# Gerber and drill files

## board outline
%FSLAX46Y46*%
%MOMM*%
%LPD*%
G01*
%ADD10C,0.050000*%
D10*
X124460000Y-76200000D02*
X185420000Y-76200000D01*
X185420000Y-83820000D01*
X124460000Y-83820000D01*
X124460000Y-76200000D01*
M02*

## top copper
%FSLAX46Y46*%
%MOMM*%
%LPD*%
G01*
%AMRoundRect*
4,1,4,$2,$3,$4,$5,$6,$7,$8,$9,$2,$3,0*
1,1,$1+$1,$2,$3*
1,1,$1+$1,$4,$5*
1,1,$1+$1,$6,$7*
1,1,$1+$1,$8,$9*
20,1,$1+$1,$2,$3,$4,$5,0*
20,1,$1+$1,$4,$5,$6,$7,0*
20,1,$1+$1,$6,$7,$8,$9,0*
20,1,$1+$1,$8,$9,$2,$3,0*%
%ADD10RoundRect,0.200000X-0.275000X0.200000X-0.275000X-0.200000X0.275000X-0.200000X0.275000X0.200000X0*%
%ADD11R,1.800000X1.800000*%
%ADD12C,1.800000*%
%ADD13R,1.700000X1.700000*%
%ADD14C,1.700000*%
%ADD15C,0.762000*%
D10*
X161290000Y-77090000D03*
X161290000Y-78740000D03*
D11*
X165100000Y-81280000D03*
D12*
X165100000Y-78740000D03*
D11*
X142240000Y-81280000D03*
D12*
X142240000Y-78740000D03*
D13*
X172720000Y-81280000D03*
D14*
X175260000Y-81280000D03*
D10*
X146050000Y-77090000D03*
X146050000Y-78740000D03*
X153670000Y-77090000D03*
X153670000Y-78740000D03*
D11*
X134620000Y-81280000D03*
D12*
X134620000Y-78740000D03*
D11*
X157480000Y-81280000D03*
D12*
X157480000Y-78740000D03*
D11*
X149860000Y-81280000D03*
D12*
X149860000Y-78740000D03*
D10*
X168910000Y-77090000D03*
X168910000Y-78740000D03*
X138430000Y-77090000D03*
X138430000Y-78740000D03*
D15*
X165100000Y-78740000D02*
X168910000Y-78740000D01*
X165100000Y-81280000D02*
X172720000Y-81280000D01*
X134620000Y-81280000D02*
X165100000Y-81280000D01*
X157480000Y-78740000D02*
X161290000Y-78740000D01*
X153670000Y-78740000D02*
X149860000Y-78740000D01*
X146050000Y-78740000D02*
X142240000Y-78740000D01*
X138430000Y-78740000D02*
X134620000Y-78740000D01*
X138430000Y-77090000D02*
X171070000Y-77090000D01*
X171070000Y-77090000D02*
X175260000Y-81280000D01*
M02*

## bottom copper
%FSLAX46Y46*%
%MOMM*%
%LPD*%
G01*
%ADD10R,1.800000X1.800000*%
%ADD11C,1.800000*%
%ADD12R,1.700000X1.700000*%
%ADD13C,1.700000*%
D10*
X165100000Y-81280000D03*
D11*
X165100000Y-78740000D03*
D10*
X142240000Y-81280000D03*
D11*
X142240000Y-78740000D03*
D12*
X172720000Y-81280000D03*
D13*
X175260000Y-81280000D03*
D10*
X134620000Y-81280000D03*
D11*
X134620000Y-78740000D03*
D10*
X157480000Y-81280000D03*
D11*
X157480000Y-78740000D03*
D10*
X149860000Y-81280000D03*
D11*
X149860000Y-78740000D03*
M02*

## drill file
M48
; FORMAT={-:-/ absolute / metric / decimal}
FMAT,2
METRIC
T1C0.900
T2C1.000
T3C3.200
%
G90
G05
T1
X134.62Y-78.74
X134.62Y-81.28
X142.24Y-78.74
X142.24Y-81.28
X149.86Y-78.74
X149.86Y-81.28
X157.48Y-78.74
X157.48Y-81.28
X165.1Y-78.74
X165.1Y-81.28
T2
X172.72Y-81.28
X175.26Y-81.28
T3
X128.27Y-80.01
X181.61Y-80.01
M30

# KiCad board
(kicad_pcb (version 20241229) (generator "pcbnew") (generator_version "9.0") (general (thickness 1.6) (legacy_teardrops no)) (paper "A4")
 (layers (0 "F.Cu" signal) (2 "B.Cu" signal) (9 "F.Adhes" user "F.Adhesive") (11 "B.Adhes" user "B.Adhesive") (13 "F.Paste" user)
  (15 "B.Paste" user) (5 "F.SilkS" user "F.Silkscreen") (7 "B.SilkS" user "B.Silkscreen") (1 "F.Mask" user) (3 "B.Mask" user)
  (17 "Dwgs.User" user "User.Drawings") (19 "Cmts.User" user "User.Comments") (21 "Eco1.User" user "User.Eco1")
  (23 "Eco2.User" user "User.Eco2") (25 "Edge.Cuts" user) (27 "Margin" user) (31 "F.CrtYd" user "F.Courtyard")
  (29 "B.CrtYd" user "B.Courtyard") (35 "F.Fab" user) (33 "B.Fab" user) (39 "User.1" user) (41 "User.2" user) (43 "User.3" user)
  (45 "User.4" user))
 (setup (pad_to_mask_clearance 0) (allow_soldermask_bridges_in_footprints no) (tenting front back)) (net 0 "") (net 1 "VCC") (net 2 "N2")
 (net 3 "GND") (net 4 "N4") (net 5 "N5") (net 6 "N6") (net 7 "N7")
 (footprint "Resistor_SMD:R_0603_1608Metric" (layer "F.Cu") (at 161.29 77.915 -90)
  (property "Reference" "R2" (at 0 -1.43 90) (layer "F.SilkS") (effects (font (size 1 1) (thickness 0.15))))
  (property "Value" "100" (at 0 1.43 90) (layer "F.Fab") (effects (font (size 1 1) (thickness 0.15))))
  (pad "1" smd roundrect (at -0.825 0 270) (size 0.8 0.95) (layers "F.Cu" "F.Mask" "F.Paste") (roundrect_rratio 0.25) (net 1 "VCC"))
  (pad "2" smd roundrect (at 0.825 0 270) (size 0.8 0.95) (layers "F.Cu" "F.Mask" "F.Paste") (roundrect_rratio 0.25) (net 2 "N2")))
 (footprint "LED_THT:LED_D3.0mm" (layer "F.Cu") (at 165.1 81.28 90)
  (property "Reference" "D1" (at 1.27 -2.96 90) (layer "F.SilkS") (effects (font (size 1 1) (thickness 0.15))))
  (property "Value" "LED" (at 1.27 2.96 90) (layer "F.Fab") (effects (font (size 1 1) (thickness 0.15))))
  (pad "1" thru_hole rect (at 0 0 90) (size 1.8 1.8) (drill 0.9) (layers "*.Cu" "*.Mask") (remove_unused_layers no) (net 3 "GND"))
  (pad "2" thru_hole circle (at 2.54 0 90) (size 1.8 1.8) (drill 0.9) (layers "*.Cu" "*.Mask") (remove_unused_layers no) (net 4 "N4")))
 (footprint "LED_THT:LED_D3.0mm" (layer "F.Cu") (at 142.24 81.28 90)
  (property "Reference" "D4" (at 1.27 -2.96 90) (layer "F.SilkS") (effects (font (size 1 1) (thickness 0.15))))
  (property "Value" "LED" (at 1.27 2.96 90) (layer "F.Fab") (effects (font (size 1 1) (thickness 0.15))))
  (pad "1" thru_hole rect (at 0 0 90) (size 1.8 1.8) (drill 0.9) (layers "*.Cu" "*.Mask") (remove_unused_layers no) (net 3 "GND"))
  (pad "2" thru_hole circle (at 2.54 0 90) (size 1.8 1.8) (drill 0.9) (layers "*.Cu" "*.Mask") (remove_unused_layers no) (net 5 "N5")))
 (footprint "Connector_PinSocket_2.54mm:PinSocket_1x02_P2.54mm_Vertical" (layer "F.Cu") (at 172.72 81.28 90)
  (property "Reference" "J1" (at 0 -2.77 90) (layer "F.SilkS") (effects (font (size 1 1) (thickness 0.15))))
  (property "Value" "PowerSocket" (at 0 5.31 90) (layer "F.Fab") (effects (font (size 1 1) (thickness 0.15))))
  (pad "1" thru_hole rect (at 0 0 90) (size 1.7 1.7) (drill 1) (layers "*.Cu" "*.Mask") (remove_unused_layers no) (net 3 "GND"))
  (pad "2" thru_hole circle (at 0 2.54 90) (size 1.7 1.7) (drill 1) (layers "*.Cu" "*.Mask") (remove_unused_layers no) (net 1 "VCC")))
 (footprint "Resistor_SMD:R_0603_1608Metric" (layer "F.Cu") (at 146.05 77.915 -90)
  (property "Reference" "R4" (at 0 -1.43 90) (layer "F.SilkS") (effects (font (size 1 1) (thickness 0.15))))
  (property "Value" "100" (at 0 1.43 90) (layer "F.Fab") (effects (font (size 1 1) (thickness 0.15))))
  (pad "1" smd roundrect (at -0.825 0 270) (size 0.8 0.95) (layers "F.Cu" "F.Mask" "F.Paste") (roundrect_rratio 0.25) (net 1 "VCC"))
  (pad "2" smd roundrect (at 0.825 0 270) (size 0.8 0.95) (layers "F.Cu" "F.Mask" "F.Paste") (roundrect_rratio 0.25) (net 5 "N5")))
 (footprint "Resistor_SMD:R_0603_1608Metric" (layer "F.Cu") (at 153.67 77.915 -90)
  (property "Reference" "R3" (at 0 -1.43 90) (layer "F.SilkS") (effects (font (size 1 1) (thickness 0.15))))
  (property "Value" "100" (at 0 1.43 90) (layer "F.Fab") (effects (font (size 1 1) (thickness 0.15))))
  (pad "1" smd roundrect (at -0.825 0 270) (size 0.8 0.95) (layers "F.Cu" "F.Mask" "F.Paste") (roundrect_rratio 0.25) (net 1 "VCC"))
  (pad "2" smd roundrect (at 0.825 0 270) (size 0.8 0.95) (layers "F.Cu" "F.Mask" "F.Paste") (roundrect_rratio 0.25) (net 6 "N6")))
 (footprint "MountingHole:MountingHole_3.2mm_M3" (layer "F.Cu") (at 128.27 80.01)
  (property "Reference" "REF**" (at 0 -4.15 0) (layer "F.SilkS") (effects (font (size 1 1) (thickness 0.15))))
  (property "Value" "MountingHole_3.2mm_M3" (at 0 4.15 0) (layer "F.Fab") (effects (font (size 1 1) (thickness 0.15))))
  (pad "" np_thru_hole circle (at 0 0) (size 3.2 3.2) (drill 3.2) (layers "*.Cu" "*.Mask")))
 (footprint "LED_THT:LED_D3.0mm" (layer "F.Cu") (at 134.62 81.28 90)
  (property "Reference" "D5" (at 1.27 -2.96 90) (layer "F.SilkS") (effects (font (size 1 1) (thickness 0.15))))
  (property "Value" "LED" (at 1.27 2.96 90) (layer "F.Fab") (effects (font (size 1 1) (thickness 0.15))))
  (pad "1" thru_hole rect (at 0 0 90) (size 1.8 1.8) (drill 0.9) (layers "*.Cu" "*.Mask") (remove_unused_layers no) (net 3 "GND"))
  (pad "2" thru_hole circle (at 2.54 0 90) (size 1.8 1.8) (drill 0.9) (layers "*.Cu" "*.Mask") (remove_unused_layers no) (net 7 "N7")))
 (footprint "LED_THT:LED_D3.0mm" (layer "F.Cu") (at 157.48 81.28 90)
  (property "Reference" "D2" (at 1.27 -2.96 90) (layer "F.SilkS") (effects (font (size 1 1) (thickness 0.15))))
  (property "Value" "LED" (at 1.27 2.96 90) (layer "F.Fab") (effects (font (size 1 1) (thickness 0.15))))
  (pad "1" thru_hole rect (at 0 0 90) (size 1.8 1.8) (drill 0.9) (layers "*.Cu" "*.Mask") (remove_unused_layers no) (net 3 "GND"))
  (pad "2" thru_hole circle (at 2.54 0 90) (size 1.8 1.8) (drill 0.9) (layers "*.Cu" "*.Mask") (remove_unused_layers no) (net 2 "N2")))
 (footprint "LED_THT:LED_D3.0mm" (layer "F.Cu") (at 149.86 81.28 90)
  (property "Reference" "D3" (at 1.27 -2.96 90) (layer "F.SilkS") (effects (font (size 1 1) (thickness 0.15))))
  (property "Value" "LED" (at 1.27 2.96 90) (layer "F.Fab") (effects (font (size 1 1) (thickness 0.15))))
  (pad "1" thru_hole rect (at 0 0 90) (size 1.8 1.8) (drill 0.9) (layers "*.Cu" "*.Mask") (remove_unused_layers no) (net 3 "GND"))
  (pad "2" thru_hole circle (at 2.54 0 90) (size 1.8 1.8) (drill 0.9) (layers "*.Cu" "*.Mask") (remove_unused_layers no) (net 6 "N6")))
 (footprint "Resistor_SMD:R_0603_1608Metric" (layer "F.Cu") (at 168.91 77.915 -90)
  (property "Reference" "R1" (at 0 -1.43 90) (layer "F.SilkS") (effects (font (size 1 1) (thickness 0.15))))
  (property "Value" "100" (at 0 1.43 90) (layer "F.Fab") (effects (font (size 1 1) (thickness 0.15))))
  (pad "1" smd roundrect (at -0.825 0 270) (size 0.8 0.95) (layers "F.Cu" "F.Mask" "F.Paste") (roundrect_rratio 0.25) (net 1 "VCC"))
  (pad "2" smd roundrect (at 0.825 0 270) (size 0.8 0.95) (layers "F.Cu" "F.Mask" "F.Paste") (roundrect_rratio 0.25) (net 4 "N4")))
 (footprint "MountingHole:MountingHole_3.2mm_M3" (layer "F.Cu") (at 181.61 80.01)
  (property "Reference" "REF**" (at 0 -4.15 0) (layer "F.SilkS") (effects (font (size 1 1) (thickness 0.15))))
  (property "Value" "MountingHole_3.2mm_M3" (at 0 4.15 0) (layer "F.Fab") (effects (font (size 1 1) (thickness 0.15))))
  (pad "" np_thru_hole circle (at 0 0) (size 3.2 3.2) (drill 3.2) (layers "*.Cu" "*.Mask")))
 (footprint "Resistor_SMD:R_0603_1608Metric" (layer "F.Cu") (at 138.43 77.915 -90)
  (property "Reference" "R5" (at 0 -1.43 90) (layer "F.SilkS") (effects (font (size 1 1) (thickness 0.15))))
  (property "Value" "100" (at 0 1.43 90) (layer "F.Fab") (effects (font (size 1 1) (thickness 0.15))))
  (pad "1" smd roundrect (at -0.825 0 270) (size 0.8 0.95) (layers "F.Cu" "F.Mask" "F.Paste") (roundrect_rratio 0.25) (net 1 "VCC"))
  (pad "2" smd roundrect (at 0.825 0 270) (size 0.8 0.95) (layers "F.Cu" "F.Mask" "F.Paste") (roundrect_rratio 0.25) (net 7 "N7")))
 (gr_rect (start 124.46 76.2) (end 185.42 83.82) (stroke (width 0.05) (type default)) (fill no) (layer "Edge.Cuts"))
 (segment (start 165.1 78.74) (end 168.91 78.74) (width 0.762) (layer "F.Cu") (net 4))
 (segment (start 165.1 81.28) (end 172.72 81.28) (width 0.762) (layer "F.Cu") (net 3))
 (segment (start 134.62 81.28) (end 165.1 81.28) (width 0.762) (layer "F.Cu") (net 3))
 (segment (start 157.48 78.74) (end 161.29 78.74) (width 0.762) (layer "F.Cu") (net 2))
 (segment (start 153.67 78.74) (end 149.86 78.74) (width 0.762) (layer "F.Cu") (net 6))
 (segment (start 146.05 78.74) (end 142.24 78.74) (width 0.762) (layer "F.Cu") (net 5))
 (segment (start 138.43 78.74) (end 134.62 78.74) (width 0.762) (layer "F.Cu") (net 7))
 (segment (start 138.43 77.09) (end 171.07 77.09) (width 0.762) (layer "F.Cu") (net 1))
 (segment (start 171.07 77.09) (end 175.26 81.28) (width 0.762) (layer "F.Cu") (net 1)))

